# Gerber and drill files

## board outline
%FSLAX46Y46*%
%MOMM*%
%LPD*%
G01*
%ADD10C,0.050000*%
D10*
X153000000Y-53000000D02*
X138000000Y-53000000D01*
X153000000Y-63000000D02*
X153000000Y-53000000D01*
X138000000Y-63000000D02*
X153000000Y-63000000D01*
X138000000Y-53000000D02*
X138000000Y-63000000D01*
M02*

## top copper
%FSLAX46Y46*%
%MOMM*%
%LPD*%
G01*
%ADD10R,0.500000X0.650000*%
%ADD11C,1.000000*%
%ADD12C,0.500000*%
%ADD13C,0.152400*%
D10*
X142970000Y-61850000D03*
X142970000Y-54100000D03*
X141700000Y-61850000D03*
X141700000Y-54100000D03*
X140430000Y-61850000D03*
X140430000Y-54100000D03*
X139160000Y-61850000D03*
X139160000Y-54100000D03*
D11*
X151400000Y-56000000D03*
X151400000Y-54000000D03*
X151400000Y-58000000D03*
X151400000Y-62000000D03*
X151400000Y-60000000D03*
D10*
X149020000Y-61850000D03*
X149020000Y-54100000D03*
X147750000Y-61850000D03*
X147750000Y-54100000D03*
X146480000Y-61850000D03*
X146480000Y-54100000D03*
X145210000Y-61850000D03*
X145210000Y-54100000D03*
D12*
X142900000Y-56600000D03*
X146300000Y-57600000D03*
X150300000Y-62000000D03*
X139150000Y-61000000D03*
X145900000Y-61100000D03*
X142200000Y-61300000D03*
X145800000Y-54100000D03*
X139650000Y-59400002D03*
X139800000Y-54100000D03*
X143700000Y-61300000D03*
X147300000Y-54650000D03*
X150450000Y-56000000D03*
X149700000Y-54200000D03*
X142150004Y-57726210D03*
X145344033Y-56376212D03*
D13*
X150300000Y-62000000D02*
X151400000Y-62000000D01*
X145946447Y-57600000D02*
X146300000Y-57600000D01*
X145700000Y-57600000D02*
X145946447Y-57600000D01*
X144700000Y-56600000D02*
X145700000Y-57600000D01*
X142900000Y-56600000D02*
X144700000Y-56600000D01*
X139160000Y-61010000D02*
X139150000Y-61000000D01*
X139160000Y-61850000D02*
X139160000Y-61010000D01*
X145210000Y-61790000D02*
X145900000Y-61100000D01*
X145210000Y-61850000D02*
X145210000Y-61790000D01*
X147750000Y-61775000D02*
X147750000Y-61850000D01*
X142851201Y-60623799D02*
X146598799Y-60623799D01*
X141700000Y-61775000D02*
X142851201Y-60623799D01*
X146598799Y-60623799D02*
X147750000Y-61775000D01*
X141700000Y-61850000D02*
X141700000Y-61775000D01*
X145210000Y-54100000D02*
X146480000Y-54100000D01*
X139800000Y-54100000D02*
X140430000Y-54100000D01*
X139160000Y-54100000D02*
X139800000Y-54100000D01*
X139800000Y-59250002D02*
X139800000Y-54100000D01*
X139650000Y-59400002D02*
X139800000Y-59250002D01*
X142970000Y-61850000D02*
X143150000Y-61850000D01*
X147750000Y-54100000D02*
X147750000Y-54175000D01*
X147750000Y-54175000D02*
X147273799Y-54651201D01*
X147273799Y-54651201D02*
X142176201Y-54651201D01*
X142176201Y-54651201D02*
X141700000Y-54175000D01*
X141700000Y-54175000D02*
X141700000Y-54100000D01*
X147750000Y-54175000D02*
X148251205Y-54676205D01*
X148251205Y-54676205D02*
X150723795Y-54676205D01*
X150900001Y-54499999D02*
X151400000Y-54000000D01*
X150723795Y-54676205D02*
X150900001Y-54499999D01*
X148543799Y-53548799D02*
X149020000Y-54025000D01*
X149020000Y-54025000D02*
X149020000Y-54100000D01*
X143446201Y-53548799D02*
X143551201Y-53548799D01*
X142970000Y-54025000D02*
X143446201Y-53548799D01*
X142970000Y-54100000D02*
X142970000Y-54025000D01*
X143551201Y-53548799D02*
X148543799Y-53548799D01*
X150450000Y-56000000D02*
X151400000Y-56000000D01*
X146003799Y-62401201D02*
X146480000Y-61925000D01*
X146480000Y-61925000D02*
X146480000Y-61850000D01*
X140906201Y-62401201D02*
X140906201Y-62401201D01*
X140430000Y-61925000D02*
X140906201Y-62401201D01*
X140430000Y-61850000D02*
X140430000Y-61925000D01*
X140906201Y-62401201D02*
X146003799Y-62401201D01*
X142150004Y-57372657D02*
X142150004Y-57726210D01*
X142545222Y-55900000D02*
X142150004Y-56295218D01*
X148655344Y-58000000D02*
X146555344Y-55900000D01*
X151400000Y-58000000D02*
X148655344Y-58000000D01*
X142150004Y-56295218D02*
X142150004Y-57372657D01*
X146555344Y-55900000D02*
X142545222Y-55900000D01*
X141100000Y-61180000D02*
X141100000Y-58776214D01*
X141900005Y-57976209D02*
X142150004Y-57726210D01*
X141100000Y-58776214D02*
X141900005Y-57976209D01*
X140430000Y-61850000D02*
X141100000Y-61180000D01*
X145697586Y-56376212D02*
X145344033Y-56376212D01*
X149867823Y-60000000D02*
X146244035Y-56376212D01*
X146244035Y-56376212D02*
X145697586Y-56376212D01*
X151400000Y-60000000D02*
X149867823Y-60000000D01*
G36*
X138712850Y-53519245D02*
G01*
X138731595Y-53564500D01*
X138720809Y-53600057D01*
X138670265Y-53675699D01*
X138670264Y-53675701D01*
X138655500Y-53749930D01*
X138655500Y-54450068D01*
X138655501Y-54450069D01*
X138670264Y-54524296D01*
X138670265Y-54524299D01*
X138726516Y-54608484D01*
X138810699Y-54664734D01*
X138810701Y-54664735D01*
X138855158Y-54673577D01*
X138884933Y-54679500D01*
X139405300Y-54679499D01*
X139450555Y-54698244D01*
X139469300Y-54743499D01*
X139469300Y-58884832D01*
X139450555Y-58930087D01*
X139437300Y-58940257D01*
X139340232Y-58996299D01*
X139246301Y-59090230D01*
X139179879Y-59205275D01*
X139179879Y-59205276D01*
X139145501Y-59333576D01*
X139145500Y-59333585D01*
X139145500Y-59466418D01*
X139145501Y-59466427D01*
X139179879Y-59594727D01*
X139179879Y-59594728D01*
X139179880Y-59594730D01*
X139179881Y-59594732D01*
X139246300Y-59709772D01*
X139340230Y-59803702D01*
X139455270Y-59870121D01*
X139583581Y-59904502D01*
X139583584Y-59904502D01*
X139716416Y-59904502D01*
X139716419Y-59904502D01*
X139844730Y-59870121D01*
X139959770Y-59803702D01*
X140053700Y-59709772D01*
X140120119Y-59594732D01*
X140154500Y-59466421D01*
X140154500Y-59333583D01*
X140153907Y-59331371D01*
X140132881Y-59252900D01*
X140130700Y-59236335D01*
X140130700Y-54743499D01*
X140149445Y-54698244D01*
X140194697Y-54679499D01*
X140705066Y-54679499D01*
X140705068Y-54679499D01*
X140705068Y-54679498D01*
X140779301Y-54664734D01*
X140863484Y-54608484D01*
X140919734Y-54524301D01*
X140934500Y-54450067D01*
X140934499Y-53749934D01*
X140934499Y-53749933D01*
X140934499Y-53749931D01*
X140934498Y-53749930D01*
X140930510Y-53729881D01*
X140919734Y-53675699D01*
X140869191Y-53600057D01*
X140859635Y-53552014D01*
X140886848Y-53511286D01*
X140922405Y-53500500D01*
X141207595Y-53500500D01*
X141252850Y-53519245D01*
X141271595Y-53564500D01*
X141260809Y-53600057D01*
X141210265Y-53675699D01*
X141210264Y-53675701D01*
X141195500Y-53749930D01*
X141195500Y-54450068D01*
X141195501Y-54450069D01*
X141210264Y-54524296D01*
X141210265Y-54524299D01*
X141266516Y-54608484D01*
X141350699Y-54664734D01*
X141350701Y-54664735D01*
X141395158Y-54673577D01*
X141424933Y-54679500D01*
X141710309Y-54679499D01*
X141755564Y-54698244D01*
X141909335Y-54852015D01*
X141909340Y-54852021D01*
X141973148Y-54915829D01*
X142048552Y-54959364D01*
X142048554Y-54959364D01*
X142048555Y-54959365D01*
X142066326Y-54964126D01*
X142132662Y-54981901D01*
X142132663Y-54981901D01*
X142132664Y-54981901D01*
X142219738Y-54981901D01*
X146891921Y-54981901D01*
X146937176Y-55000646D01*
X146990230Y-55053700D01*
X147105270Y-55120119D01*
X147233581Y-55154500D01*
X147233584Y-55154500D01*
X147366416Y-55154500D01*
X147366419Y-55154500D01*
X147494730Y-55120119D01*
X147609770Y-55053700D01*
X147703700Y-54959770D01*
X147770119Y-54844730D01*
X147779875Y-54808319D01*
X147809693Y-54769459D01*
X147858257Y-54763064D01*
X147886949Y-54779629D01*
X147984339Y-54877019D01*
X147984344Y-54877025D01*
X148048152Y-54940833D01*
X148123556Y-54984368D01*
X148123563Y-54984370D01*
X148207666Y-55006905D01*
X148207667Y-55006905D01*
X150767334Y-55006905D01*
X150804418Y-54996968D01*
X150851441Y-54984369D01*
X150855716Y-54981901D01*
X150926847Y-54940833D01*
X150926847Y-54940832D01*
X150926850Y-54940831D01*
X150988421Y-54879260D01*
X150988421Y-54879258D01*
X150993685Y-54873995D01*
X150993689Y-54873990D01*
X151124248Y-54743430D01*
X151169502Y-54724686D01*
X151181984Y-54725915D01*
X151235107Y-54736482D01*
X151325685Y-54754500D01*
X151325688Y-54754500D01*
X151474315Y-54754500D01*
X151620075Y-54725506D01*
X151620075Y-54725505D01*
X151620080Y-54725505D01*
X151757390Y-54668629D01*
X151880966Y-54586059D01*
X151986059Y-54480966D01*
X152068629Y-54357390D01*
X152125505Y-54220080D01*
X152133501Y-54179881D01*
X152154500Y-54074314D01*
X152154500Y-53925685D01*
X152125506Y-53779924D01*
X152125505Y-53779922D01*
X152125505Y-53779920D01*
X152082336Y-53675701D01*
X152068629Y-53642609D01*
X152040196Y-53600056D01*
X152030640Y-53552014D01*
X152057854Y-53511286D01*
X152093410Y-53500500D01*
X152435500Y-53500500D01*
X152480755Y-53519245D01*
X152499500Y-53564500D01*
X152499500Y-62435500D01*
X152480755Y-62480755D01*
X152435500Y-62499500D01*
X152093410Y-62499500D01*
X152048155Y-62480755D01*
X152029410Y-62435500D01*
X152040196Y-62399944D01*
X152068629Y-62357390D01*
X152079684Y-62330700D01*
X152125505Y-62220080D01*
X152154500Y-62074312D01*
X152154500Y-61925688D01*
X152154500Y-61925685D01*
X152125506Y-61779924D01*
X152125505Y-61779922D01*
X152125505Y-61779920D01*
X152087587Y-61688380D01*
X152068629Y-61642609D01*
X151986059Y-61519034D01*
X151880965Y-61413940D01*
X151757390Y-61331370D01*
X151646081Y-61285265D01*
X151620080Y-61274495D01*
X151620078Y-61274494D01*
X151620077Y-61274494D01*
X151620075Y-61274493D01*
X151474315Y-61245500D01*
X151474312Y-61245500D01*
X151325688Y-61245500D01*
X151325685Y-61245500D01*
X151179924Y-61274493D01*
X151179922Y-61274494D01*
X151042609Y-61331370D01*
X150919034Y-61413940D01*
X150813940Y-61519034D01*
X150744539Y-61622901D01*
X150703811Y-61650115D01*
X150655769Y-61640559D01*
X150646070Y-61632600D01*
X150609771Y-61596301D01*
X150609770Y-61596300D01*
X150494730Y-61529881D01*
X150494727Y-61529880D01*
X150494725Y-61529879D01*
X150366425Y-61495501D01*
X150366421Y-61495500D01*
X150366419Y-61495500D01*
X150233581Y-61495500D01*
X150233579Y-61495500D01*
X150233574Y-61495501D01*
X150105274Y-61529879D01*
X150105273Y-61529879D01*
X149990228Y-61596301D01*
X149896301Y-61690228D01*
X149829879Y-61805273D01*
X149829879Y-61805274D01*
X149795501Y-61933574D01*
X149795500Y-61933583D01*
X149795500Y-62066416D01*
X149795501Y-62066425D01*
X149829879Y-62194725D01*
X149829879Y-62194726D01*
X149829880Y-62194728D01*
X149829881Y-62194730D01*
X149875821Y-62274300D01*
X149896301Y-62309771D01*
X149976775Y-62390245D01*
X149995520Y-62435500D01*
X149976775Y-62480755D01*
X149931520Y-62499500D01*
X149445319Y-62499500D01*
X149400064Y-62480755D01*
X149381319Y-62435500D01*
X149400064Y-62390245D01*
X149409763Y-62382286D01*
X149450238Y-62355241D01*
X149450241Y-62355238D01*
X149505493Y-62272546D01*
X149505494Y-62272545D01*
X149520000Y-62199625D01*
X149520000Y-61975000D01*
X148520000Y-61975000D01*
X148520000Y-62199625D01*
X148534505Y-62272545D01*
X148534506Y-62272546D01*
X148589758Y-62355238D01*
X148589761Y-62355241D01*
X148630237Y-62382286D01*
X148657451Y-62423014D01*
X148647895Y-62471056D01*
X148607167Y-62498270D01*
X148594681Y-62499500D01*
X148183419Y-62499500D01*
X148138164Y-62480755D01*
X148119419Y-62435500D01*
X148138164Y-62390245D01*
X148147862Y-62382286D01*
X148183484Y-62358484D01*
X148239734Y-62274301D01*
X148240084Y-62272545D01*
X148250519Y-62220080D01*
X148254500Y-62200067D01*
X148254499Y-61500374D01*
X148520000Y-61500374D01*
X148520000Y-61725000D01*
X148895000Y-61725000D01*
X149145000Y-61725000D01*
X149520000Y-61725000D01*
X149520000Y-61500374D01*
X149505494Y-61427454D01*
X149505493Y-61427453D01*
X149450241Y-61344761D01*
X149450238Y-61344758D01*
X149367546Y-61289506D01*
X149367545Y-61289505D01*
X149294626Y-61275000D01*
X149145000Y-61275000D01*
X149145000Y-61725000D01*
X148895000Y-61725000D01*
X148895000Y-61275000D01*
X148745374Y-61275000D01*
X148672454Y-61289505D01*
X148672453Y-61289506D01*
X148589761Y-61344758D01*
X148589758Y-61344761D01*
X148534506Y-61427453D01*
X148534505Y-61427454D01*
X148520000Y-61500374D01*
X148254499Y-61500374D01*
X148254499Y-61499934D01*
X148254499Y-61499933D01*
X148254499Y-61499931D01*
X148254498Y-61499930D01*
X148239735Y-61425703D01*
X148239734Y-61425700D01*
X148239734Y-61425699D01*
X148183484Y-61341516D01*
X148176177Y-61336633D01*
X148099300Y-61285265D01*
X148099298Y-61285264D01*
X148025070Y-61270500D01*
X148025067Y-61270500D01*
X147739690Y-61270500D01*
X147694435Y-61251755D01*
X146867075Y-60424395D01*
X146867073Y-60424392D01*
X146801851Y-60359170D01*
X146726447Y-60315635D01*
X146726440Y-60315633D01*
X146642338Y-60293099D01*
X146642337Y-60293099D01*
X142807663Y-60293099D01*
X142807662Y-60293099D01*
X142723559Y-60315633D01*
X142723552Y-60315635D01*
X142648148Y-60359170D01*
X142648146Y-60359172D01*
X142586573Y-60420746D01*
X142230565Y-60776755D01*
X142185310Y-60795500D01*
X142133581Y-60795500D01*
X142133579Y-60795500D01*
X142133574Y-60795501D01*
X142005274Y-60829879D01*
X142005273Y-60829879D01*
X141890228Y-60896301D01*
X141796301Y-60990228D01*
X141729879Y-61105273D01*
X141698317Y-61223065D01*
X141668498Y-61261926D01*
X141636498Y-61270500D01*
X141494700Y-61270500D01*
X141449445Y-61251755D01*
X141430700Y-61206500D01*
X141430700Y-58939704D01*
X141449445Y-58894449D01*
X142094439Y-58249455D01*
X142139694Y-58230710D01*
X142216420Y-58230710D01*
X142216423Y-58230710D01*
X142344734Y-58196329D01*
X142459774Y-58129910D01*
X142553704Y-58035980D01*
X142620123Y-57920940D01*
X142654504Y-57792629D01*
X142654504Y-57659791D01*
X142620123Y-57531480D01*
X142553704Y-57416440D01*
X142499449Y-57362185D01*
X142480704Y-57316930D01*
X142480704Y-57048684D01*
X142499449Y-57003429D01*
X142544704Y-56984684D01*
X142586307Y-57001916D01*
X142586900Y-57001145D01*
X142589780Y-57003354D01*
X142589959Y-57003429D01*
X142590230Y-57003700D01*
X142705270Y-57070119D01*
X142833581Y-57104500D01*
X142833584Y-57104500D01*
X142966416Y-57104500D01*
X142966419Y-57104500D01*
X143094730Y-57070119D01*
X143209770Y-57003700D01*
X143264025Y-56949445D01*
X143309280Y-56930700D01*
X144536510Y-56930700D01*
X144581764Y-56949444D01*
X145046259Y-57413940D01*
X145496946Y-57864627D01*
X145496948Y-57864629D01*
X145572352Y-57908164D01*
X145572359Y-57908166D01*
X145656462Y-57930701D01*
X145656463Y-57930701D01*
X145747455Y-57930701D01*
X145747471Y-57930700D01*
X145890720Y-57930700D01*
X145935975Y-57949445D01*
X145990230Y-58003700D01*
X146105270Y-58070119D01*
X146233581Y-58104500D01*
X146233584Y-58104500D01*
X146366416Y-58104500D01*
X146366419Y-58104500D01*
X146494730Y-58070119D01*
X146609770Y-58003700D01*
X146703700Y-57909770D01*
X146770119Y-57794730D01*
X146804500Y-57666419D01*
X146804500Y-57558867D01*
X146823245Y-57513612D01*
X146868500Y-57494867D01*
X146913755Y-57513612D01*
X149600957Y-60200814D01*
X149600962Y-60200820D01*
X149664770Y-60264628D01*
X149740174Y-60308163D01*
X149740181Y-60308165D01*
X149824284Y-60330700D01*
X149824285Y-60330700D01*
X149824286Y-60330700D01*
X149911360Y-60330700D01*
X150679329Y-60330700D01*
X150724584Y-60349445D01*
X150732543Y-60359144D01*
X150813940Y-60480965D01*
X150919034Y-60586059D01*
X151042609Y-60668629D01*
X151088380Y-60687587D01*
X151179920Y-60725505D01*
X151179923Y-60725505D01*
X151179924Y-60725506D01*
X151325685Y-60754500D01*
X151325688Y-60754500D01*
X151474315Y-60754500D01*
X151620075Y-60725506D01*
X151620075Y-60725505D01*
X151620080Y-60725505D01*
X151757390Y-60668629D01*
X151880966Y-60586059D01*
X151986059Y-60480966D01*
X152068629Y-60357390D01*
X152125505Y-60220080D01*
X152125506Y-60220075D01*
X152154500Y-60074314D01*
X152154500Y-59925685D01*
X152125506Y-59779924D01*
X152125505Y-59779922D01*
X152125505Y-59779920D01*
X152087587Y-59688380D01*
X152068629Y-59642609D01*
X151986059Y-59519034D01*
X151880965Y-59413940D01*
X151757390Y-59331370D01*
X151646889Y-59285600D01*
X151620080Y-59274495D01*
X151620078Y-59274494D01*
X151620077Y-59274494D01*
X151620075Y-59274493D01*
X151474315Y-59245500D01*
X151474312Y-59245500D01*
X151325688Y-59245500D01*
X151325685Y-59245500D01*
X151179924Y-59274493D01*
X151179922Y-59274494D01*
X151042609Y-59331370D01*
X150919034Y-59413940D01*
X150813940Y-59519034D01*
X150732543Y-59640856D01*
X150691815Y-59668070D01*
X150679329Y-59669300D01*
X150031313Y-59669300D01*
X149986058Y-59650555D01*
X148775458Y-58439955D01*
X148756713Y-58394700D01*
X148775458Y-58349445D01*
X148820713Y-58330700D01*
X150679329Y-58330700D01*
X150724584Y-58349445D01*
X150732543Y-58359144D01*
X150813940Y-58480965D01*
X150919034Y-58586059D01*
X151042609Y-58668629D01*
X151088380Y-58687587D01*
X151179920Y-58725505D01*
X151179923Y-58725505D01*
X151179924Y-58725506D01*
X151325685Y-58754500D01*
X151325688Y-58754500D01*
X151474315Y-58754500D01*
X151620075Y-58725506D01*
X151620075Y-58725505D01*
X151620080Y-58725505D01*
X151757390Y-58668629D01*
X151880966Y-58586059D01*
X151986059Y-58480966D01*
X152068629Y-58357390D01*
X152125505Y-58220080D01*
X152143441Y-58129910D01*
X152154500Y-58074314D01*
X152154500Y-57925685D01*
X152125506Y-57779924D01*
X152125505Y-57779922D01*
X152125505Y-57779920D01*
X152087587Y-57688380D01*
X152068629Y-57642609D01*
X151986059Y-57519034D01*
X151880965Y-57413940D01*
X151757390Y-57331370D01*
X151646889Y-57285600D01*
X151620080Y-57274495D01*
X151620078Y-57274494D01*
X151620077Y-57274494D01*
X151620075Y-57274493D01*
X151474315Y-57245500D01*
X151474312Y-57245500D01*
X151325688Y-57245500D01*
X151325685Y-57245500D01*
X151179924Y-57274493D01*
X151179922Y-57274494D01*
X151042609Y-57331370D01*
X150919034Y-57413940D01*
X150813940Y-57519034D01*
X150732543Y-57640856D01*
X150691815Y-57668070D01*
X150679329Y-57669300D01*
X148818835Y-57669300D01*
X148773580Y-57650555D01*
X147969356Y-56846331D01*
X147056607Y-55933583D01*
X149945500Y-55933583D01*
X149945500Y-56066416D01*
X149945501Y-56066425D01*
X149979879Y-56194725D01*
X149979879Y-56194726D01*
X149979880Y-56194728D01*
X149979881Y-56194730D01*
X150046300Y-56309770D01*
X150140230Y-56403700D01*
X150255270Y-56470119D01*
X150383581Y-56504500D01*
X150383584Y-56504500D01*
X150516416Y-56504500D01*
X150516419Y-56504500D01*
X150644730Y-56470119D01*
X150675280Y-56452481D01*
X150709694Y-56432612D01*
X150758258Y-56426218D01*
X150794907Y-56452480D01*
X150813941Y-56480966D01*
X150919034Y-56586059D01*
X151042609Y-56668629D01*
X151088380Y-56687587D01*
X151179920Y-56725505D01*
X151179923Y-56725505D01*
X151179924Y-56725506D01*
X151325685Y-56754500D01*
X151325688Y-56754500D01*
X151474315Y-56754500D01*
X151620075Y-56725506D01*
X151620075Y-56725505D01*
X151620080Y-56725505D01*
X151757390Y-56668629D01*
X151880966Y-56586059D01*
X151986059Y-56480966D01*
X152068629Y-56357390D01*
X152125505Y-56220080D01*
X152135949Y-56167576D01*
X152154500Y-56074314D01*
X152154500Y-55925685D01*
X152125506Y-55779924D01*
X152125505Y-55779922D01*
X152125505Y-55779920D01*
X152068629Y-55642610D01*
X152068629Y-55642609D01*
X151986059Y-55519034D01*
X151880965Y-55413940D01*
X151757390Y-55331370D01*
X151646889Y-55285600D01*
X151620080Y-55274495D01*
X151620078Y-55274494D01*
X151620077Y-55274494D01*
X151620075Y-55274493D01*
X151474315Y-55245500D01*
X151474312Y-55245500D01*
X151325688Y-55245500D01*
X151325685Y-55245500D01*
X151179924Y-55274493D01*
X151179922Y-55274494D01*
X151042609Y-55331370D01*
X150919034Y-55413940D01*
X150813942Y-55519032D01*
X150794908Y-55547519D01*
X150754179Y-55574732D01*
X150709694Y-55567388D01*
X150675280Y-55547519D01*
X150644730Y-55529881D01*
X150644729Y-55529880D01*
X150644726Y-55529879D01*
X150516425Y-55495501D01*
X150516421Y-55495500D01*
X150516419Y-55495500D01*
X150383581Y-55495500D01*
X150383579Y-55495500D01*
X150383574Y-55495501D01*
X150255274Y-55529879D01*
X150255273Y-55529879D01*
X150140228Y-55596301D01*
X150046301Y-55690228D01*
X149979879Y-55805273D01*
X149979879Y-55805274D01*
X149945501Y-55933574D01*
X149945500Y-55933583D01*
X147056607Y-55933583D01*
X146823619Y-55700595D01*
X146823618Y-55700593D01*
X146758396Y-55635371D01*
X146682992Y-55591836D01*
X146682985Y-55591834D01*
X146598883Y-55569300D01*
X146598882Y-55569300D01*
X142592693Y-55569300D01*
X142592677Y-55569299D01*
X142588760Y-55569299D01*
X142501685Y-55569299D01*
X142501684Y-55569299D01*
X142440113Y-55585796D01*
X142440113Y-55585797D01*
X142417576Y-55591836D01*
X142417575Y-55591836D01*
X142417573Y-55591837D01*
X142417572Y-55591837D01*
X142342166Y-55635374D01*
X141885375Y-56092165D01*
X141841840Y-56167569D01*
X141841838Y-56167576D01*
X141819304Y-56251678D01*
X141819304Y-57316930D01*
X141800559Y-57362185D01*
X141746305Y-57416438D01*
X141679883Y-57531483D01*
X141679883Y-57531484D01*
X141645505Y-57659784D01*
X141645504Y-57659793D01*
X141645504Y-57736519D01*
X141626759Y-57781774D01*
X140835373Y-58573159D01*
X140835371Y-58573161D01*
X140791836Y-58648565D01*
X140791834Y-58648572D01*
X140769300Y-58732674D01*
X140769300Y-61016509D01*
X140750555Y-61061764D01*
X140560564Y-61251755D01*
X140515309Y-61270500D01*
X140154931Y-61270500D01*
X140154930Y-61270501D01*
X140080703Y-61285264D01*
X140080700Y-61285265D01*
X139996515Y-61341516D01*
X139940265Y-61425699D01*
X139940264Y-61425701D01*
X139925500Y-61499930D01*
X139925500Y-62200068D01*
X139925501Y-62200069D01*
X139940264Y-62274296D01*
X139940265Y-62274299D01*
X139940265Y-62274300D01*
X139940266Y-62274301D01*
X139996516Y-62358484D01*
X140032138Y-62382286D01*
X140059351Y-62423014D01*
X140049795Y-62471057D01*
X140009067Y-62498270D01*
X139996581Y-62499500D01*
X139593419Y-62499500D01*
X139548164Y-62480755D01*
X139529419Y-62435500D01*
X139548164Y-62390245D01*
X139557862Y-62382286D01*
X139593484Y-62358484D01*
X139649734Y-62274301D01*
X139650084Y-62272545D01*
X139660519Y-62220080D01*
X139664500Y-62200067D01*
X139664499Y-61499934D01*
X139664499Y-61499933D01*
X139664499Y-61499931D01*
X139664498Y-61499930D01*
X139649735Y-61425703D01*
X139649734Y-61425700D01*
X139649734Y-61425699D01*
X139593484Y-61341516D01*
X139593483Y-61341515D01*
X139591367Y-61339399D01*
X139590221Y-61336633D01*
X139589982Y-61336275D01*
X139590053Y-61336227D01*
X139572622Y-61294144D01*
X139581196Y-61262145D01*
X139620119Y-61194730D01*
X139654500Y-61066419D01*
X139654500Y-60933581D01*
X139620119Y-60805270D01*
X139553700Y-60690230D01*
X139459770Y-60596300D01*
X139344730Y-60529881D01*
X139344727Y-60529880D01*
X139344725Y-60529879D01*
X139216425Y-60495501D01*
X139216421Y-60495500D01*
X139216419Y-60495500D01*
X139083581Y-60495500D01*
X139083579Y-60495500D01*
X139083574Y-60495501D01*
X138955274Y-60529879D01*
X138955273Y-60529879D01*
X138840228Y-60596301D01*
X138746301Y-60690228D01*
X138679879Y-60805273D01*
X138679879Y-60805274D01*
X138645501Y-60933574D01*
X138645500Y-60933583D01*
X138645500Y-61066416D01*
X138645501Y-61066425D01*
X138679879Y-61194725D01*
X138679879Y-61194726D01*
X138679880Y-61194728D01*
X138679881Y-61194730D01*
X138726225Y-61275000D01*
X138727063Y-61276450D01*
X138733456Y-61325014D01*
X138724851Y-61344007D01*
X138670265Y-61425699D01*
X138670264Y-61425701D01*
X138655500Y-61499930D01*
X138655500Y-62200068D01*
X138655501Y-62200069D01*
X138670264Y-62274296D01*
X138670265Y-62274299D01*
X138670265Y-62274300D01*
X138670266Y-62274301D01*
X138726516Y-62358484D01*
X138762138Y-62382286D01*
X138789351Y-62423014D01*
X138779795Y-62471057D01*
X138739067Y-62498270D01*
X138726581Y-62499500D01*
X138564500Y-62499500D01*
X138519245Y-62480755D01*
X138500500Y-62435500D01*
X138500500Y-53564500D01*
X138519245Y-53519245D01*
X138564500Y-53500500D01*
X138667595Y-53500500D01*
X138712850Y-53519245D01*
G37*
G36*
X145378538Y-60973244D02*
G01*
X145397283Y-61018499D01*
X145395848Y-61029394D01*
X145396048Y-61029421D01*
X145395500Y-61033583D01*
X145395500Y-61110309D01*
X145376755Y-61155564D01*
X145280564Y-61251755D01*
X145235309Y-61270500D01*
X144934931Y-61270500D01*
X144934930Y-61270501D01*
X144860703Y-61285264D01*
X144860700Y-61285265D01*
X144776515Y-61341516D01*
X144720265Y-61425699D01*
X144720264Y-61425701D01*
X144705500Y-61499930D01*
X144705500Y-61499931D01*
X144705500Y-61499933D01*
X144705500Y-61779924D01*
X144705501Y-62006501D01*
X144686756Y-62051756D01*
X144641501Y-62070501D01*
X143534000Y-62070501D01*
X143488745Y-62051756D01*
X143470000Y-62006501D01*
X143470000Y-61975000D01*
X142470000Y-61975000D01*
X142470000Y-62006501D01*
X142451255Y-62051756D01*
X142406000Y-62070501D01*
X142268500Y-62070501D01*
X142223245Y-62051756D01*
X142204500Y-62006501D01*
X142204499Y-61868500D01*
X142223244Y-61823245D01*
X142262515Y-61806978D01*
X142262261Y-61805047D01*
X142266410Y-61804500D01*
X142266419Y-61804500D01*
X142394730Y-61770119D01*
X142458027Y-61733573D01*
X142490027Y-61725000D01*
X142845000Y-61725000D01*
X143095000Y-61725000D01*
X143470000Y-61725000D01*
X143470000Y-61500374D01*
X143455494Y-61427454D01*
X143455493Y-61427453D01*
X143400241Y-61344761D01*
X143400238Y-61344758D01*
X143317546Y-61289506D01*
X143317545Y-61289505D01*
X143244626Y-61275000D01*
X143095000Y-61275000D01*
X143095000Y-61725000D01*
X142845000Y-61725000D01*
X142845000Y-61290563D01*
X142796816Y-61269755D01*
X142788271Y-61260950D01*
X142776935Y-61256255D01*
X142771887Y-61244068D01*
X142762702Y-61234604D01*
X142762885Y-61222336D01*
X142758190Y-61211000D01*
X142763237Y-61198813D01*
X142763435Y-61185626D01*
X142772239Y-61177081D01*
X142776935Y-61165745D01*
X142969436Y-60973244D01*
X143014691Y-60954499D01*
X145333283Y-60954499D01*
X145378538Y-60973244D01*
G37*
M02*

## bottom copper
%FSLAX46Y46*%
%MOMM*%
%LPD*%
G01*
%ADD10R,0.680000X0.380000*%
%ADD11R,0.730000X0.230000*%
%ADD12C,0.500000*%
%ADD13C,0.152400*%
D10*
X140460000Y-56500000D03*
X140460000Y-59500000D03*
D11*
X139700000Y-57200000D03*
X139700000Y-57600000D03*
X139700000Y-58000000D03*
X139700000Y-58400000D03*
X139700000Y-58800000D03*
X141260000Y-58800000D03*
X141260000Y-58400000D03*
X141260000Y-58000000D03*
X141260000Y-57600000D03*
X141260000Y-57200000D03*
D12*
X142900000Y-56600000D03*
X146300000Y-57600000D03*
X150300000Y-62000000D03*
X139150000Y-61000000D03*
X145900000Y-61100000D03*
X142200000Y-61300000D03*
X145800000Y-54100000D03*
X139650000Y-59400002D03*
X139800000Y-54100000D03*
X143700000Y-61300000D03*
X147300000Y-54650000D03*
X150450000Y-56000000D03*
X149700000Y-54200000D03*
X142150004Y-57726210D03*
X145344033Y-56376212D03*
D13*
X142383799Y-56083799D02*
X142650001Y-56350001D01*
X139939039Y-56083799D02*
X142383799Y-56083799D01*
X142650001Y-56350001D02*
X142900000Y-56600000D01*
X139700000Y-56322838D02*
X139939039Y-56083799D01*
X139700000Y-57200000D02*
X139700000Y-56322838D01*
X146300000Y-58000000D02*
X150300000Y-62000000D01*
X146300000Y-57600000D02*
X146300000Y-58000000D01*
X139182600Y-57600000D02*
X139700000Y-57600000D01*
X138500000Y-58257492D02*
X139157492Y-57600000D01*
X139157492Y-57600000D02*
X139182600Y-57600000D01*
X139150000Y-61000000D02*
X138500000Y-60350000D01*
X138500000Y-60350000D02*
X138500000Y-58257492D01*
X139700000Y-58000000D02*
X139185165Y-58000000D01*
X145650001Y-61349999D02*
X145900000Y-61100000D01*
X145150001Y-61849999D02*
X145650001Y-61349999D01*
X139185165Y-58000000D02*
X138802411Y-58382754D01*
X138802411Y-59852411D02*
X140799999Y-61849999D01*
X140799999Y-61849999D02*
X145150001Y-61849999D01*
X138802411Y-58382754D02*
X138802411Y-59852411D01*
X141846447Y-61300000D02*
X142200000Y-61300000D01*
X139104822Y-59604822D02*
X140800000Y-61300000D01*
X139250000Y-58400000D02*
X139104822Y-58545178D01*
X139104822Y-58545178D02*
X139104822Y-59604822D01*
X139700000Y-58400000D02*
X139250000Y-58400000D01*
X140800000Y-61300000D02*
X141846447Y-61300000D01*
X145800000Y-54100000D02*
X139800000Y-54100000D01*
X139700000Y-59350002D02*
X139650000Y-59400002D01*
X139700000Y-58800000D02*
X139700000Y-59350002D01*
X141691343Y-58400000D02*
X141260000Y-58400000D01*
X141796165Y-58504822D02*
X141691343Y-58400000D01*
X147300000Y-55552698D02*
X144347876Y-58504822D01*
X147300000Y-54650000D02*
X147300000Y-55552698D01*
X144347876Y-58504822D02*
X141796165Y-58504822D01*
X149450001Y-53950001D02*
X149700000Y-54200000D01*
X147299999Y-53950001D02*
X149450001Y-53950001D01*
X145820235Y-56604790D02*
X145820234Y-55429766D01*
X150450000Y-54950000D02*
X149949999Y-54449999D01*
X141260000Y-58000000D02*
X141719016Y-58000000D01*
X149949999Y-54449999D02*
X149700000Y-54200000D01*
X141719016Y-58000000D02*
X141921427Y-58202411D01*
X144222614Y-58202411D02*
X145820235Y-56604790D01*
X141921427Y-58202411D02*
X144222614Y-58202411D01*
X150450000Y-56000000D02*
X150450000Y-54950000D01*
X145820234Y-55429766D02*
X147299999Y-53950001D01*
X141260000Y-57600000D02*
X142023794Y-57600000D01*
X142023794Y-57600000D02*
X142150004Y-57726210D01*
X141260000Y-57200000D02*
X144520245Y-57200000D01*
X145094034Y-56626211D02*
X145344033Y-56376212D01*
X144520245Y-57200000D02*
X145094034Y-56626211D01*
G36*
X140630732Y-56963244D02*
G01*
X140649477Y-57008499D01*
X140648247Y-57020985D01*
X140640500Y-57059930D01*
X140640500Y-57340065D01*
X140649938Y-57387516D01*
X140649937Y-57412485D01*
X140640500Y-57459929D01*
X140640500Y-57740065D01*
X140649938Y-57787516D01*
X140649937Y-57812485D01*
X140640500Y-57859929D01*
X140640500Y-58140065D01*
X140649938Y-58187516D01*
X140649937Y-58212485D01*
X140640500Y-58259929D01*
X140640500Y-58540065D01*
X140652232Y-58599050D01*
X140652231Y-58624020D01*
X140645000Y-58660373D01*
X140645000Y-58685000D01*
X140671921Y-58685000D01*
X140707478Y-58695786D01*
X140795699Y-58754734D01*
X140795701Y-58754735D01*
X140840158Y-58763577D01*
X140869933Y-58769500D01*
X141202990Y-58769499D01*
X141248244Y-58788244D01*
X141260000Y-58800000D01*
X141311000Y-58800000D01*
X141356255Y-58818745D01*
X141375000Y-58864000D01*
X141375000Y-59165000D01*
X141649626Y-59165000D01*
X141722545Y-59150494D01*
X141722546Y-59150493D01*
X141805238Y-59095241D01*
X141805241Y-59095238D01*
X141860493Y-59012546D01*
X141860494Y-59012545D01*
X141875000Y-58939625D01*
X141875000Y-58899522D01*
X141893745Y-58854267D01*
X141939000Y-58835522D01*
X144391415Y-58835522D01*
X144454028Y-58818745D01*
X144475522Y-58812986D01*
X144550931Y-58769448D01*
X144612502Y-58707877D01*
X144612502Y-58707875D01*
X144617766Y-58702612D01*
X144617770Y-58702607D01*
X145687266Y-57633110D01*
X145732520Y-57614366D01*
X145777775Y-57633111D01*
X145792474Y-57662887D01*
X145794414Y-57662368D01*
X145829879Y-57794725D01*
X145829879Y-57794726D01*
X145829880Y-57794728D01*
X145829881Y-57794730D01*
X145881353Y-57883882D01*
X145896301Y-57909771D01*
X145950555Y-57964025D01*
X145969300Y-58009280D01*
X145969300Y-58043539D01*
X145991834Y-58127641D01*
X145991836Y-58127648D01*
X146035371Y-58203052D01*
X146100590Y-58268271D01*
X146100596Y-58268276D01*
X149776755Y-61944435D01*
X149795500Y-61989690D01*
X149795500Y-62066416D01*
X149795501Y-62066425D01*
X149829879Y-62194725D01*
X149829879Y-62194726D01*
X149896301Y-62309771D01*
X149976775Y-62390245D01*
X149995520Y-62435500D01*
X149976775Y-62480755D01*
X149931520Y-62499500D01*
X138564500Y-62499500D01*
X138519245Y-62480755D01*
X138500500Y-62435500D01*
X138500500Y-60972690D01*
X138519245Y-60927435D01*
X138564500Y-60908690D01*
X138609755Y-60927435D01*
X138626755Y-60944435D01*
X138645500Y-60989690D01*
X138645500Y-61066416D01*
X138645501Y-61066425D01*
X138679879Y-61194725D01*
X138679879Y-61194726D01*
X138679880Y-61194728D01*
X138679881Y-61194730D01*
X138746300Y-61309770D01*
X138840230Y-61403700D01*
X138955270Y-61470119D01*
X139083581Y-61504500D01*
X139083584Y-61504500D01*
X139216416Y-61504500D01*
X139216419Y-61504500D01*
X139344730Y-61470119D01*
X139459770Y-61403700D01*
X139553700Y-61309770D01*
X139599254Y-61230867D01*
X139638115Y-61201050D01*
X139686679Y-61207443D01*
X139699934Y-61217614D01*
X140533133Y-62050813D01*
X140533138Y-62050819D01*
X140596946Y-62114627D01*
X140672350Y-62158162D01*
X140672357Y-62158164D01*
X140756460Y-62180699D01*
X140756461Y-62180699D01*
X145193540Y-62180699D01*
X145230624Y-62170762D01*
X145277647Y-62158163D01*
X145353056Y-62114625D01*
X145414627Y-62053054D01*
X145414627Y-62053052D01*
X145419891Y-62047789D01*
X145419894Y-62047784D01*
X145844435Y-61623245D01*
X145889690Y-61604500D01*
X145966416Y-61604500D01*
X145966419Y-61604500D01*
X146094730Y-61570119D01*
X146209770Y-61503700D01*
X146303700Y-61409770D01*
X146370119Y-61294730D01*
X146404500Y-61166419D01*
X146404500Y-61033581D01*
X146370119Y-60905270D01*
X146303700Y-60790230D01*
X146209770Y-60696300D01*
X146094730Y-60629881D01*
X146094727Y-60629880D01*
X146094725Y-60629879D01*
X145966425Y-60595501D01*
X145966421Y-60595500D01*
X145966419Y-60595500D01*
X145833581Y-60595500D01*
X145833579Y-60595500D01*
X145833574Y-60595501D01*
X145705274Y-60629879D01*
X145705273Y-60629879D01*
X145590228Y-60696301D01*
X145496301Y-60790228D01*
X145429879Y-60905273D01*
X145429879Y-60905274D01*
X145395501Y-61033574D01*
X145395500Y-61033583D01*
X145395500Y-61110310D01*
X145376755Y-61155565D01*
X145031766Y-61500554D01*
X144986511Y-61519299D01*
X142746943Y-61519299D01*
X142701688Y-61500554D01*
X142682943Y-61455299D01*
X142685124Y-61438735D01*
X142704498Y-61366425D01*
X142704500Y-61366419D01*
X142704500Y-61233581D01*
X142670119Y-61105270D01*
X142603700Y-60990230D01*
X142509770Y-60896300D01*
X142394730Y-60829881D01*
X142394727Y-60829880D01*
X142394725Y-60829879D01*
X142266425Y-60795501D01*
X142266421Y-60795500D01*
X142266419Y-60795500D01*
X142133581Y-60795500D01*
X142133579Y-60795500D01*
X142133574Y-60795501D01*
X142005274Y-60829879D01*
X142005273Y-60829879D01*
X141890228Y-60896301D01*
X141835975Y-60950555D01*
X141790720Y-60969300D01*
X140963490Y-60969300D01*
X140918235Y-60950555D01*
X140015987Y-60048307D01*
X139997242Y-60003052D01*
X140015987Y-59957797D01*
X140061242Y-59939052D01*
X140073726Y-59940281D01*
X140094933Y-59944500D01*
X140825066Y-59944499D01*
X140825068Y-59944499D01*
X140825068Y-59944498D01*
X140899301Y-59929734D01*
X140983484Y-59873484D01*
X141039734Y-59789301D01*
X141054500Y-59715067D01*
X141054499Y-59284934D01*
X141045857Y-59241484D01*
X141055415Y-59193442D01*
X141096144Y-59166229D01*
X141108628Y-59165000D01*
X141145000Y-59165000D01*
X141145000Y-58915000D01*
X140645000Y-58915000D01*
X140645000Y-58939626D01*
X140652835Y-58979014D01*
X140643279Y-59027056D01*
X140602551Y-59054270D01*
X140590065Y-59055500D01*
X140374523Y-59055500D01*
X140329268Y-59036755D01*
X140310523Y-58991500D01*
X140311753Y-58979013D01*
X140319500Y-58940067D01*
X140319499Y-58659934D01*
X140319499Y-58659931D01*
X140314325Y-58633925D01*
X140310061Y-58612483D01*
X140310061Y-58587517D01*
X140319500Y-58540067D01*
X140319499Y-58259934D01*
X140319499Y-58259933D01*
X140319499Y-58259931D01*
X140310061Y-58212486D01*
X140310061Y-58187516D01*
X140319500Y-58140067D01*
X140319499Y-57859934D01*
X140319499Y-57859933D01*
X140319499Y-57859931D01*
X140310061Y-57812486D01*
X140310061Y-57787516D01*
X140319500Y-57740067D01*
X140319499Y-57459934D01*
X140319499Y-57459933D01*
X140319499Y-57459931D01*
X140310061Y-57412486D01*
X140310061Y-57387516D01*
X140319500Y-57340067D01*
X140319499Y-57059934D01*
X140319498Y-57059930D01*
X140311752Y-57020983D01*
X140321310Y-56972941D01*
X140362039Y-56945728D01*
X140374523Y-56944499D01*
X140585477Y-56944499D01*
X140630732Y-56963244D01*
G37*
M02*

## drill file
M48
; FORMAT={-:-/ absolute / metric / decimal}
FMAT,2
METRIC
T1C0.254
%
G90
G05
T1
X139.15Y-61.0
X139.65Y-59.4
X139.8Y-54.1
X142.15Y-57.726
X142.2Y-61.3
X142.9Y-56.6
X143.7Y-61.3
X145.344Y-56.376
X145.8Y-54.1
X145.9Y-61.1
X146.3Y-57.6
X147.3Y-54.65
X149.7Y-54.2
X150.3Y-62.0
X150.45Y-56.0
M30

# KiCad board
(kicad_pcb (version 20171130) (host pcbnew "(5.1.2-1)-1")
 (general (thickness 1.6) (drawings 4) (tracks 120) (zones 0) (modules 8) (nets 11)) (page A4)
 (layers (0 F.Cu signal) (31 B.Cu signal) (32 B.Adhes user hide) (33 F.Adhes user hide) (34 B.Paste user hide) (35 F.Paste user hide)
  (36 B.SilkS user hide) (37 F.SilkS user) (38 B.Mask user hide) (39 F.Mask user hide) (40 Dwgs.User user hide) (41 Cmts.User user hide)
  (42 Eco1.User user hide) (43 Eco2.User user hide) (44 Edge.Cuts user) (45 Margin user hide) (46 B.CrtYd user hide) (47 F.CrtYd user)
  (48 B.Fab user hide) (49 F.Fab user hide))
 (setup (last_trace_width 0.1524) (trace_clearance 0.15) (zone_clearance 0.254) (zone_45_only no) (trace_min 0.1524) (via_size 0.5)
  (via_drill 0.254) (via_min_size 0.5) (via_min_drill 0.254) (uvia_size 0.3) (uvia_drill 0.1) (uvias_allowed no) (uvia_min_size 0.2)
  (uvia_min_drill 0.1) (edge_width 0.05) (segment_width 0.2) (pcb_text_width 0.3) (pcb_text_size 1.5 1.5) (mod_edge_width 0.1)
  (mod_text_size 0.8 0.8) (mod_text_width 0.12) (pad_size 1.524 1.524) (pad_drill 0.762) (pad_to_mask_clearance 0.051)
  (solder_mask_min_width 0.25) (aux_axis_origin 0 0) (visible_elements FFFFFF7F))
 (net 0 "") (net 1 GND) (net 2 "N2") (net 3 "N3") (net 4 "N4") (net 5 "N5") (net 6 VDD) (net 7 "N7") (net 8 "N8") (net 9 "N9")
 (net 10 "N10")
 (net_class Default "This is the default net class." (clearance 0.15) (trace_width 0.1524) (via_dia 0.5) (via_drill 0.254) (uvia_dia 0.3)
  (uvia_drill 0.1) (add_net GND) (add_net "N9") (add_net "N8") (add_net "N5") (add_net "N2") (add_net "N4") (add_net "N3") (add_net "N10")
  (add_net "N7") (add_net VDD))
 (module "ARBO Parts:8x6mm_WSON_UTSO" (layer F.Cu) (at 141.065 57.975)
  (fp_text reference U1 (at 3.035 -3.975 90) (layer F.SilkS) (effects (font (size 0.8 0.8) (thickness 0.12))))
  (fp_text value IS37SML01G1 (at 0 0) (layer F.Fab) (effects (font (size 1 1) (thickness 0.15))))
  (pad 4 smd rect (at 1.905 3.875) (size 0.5 0.65) (layers F.Cu F.Paste F.Mask) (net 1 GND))
  (pad 5 smd rect (at 1.905 -3.875) (size 0.5 0.65) (layers F.Cu F.Paste F.Mask) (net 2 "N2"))
  (pad 3 smd rect (at 0.635 3.875) (size 0.5 0.65) (layers F.Cu F.Paste F.Mask) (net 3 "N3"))
  (pad 6 smd rect (at 0.635 -3.875) (size 0.5 0.65) (layers F.Cu F.Paste F.Mask) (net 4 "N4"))
  (pad 2 smd rect (at -0.635 3.875) (size 0.5 0.65) (layers F.Cu F.Paste F.Mask) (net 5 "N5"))
  (pad 7 smd rect (at -0.635 -3.875) (size 0.5 0.65) (layers F.Cu F.Paste F.Mask) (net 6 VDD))
  (pad 1 smd rect (at -1.905 3.875) (size 0.5 0.65) (layers F.Cu F.Paste F.Mask) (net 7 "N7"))
  (pad 8 smd rect (at -1.905 -3.875) (size 0.5 0.65) (layers F.Cu F.Paste F.Mask) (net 6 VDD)))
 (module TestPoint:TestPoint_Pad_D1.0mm (layer F.Cu) (at 151.4 56)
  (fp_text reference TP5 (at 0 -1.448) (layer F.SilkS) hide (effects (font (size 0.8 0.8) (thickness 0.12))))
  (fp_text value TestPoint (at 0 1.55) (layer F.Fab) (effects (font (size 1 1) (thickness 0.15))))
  (pad 1 smd circle (at 0 0) (size 1 1) (layers F.Cu F.Mask) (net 2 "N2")))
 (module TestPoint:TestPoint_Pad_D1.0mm (layer F.Cu) (at 151.4 54)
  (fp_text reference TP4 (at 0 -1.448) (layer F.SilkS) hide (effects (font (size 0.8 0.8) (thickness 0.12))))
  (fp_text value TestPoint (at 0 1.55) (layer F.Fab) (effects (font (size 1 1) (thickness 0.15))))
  (pad 1 smd circle (at 0 0) (size 1 1) (layers F.Cu F.Mask) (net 4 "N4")))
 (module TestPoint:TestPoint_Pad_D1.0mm (layer F.Cu) (at 151.4 58)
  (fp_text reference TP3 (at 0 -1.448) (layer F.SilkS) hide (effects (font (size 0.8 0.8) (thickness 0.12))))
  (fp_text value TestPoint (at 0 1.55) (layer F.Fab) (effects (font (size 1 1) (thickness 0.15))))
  (pad 1 smd circle (at 0 0) (size 1 1) (layers F.Cu F.Mask) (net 5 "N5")))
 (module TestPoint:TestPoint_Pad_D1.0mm (layer F.Cu) (at 151.4 62)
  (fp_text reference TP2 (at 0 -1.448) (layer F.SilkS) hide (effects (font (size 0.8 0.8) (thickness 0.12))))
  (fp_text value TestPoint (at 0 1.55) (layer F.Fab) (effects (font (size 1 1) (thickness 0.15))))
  (pad 1 smd circle (at 0 0) (size 1 1) (layers F.Cu F.Mask) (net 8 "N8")))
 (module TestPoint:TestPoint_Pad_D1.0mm (layer F.Cu) (at 151.4 60)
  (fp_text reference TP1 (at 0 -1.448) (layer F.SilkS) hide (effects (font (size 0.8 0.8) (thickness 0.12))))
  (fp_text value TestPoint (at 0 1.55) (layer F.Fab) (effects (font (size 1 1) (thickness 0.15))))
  (pad 1 smd circle (at 0 0) (size 1 1) (layers F.Cu F.Mask) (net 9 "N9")))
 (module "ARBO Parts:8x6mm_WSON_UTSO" (layer F.Cu) (at 147.115 57.975)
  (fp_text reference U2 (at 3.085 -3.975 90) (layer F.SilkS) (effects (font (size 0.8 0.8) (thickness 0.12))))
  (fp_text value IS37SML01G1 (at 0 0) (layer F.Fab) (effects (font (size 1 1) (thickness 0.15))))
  (pad 4 smd rect (at 1.905 3.875) (size 0.5 0.65) (layers F.Cu F.Paste F.Mask) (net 1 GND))
  (pad 5 smd rect (at 1.905 -3.875) (size 0.5 0.65) (layers F.Cu F.Paste F.Mask) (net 2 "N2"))
  (pad 3 smd rect (at 0.635 3.875) (size 0.5 0.65) (layers F.Cu F.Paste F.Mask) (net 3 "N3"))
  (pad 6 smd rect (at 0.635 -3.875) (size 0.5 0.65) (layers F.Cu F.Paste F.Mask) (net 4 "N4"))
  (pad 2 smd rect (at -0.635 3.875) (size 0.5 0.65) (layers F.Cu F.Paste F.Mask) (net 5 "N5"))
  (pad 7 smd rect (at -0.635 -3.875) (size 0.5 0.65) (layers F.Cu F.Paste F.Mask) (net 6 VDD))
  (pad 1 smd rect (at -1.905 3.875) (size 0.5 0.65) (layers F.Cu F.Paste F.Mask) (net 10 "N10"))
  (pad 8 smd rect (at -1.905 -3.875) (size 0.5 0.65) (layers F.Cu F.Paste F.Mask) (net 6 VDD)))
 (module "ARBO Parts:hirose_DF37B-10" (layer B.Cu) (at 141.26 58 270)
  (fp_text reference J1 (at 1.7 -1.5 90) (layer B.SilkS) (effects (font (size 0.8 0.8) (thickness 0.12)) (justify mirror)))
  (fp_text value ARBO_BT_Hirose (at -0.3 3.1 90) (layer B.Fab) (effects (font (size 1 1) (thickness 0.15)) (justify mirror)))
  (pad 12 smd rect (at -1.5 0.8 270) (size 0.38 0.68) (layers B.Cu B.Paste B.Mask))
  (pad 11 smd rect (at 1.5 0.8 270) (size 0.38 0.68) (layers B.Cu B.Paste B.Mask))
  (pad 10 smd rect (at -0.8 1.56 270) (size 0.23 0.73) (layers B.Cu B.Paste B.Mask) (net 8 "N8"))
  (pad 9 smd rect (at -0.4 1.56 270) (size 0.23 0.73) (layers B.Cu B.Paste B.Mask) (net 7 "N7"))
  (pad 8 smd rect (at 0 1.56 270) (size 0.23 0.73) (layers B.Cu B.Paste B.Mask) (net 10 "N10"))
  (pad 7 smd rect (at 0.4 1.56 270) (size 0.23 0.73) (layers B.Cu B.Paste B.Mask) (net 3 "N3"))
  (pad 6 smd rect (at 0.8 1.56 270) (size 0.23 0.73) (layers B.Cu B.Paste B.Mask) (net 6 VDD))
  (pad 5 smd rect (at 0.8 0 270) (size 0.23 0.73) (layers B.Cu B.Paste B.Mask) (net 1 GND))
  (pad 4 smd rect (at 0.4 0 270) (size 0.23 0.73) (layers B.Cu B.Paste B.Mask) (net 4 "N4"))
  (pad 3 smd rect (at 0 0 270) (size 0.23 0.73) (layers B.Cu B.Paste B.Mask) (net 2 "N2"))
  (pad 2 smd rect (at -0.4 0 270) (size 0.23 0.73) (layers B.Cu B.Paste B.Mask) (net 5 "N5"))
  (pad 1 smd rect (at -0.8 0 270) (size 0.23 0.73) (layers B.Cu B.Paste B.Mask) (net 9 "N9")))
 (gr_line (start 153 53) (end 138 53) (layer Edge.Cuts) (width 0.05))
 (gr_line (start 153 63) (end 153 53) (layer Edge.Cuts) (width 0.05))
 (gr_line (start 138 63) (end 153 63) (layer Edge.Cuts) (width 0.05))
 (gr_line (start 138 53) (end 138 63) (layer Edge.Cuts) (width 0.05))
 (via (at 142.9 56.6) (size 0.5) (drill 0.254) (layers F.Cu B.Cu) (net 8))
 (via (at 146.3 57.6) (size 0.5) (drill 0.254) (layers F.Cu B.Cu) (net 8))
 (via (at 150.3 62) (size 0.5) (drill 0.254) (layers F.Cu B.Cu) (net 8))
 (segment (start 150.3 62) (end 151.4 62) (width 0.1524) (layer F.Cu) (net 8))
 (segment (start 145.946447 57.6) (end 146.3 57.6) (width 0.1524) (layer F.Cu) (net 8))
 (segment (start 145.7 57.6) (end 145.946447 57.6) (width 0.1524) (layer F.Cu) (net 8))
 (segment (start 144.7 56.6) (end 145.7 57.6) (width 0.1524) (layer F.Cu) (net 8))
 (segment (start 142.9 56.6) (end 144.7 56.6) (width 0.1524) (layer F.Cu) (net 8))
 (segment (start 142.383799 56.083799) (end 142.650001 56.350001) (width 0.1524) (layer B.Cu) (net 8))
 (segment (start 139.939039 56.083799) (end 142.383799 56.083799) (width 0.1524) (layer B.Cu) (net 8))
 (segment (start 142.650001 56.350001) (end 142.9 56.6) (width 0.1524) (layer B.Cu) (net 8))
 (segment (start 139.7 56.322838) (end 139.939039 56.083799) (width 0.1524) (layer B.Cu) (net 8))
 (segment (start 139.7 57.2) (end 139.7 56.322838) (width 0.1524) (layer B.Cu) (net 8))
 (segment (start 146.3 58) (end 150.3 62) (width 0.1524) (layer B.Cu) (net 8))
 (segment (start 146.3 57.6) (end 146.3 58) (width 0.1524) (layer B.Cu) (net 8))
 (via (at 139.15 61) (size 0.5) (drill 0.254) (layers F.Cu B.Cu) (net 7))
 (segment (start 139.16 61.01) (end 139.15 61) (width 0.1524) (layer F.Cu) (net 7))
 (segment (start 139.16 61.85) (end 139.16 61.01) (width 0.1524) (layer F.Cu) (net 7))
 (segment (start 139.1826 57.6) (end 139.7 57.6) (width 0.1524) (layer B.Cu) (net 7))
 (segment (start 138.5 58.257492) (end 139.157492 57.6) (width 0.1524) (layer B.Cu) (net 7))
 (segment (start 139.157492 57.6) (end 139.1826 57.6) (width 0.1524) (layer B.Cu) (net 7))
 (segment (start 139.15 61) (end 138.5 60.35) (width 0.1524) (layer B.Cu) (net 7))
 (segment (start 138.5 60.35) (end 138.5 58.257492) (width 0.1524) (layer B.Cu) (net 7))
 (via (at 145.9 61.1) (size 0.5) (drill 0.254) (layers F.Cu B.Cu) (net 10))
 (segment (start 139.7 58) (end 139.185165 58) (width 0.1524) (layer B.Cu) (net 10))
 (segment (start 145.650001 61.349999) (end 145.9 61.1) (width 0.1524) (layer B.Cu) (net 10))
 (segment (start 145.150001 61.849999) (end 145.650001 61.349999) (width 0.1524) (layer B.Cu) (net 10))
 (segment (start 139.185165 58) (end 138.802411 58.382754) (width 0.1524) (layer B.Cu) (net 10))
 (segment (start 138.802411 59.852411) (end 140.799999 61.849999) (width 0.1524) (layer B.Cu) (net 10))
 (segment (start 140.799999 61.849999) (end 145.150001 61.849999) (width 0.1524) (layer B.Cu) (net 10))
 (segment (start 138.802411 58.382754) (end 138.802411 59.852411) (width 0.1524) (layer B.Cu) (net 10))
 (segment (start 145.21 61.79) (end 145.9 61.1) (width 0.1524) (layer F.Cu) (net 10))
 (segment (start 145.21 61.85) (end 145.21 61.79) (width 0.1524) (layer F.Cu) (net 10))
 (via (at 142.2 61.3) (size 0.5) (drill 0.254) (layers F.Cu B.Cu) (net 3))
 (segment (start 141.846447 61.3) (end 142.2 61.3) (width 0.1524) (layer B.Cu) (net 3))
 (segment (start 139.104822 59.604822) (end 140.8 61.3) (width 0.1524) (layer B.Cu) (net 3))
 (segment (start 139.25 58.4) (end 139.104822 58.545178) (width 0.1524) (layer B.Cu) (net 3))
 (segment (start 139.104822 58.545178) (end 139.104822 59.604822) (width 0.1524) (layer B.Cu) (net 3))
 (segment (start 139.7 58.4) (end 139.25 58.4) (width 0.1524) (layer B.Cu) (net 3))
 (segment (start 140.8 61.3) (end 141.846447 61.3) (width 0.1524) (layer B.Cu) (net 3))
 (segment (start 147.75 61.775) (end 147.75 61.85) (width 0.1524) (layer F.Cu) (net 3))
 (segment (start 142.851201 60.623799) (end 146.598799 60.623799) (width 0.1524) (layer F.Cu) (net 3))
 (segment (start 141.7 61.775) (end 142.851201 60.623799) (width 0.1524) (layer F.Cu) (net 3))
 (segment (start 146.598799 60.623799) (end 147.75 61.775) (width 0.1524) (layer F.Cu) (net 3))
 (segment (start 141.7 61.85) (end 141.7 61.775) (width 0.1524) (layer F.Cu) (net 3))
 (via (at 145.8 54.1) (size 0.5) (drill 0.254) (layers F.Cu B.Cu) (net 6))
 (segment (start 145.21 54.1) (end 146.48 54.1) (width 0.1524) (layer F.Cu) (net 6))
 (segment (start 145.8 54.1) (end 139.8 54.1) (width 0.1524) (layer B.Cu) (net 6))
 (segment (start 139.7 59.350002) (end 139.65 59.400002) (width 0.1524) (layer B.Cu) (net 6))
 (via (at 139.65 59.400002) (size 0.5) (drill 0.254) (layers F.Cu B.Cu) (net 6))
 (segment (start 139.7 58.8) (end 139.7 59.350002) (width 0.1524) (layer B.Cu) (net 6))
 (segment (start 139.8 54.1) (end 140.43 54.1) (width 0.1524) (layer F.Cu) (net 6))
 (segment (start 139.16 54.1) (end 139.8 54.1) (width 0.1524) (layer F.Cu) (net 6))
 (via (at 139.8 54.1) (size 0.5) (drill 0.254) (layers F.Cu B.Cu) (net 6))
 (segment (start 139.8 59.250002) (end 139.8 54.1) (width 0.1524) (layer F.Cu) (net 6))
 (segment (start 139.65 59.400002) (end 139.8 59.250002) (width 0.1524) (layer F.Cu) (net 6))
 (via (at 143.7 61.3) (size 0.5) (drill 0.254) (layers F.Cu B.Cu) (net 1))
 (segment (start 142.97 61.85) (end 143.15 61.85) (width 0.1524) (layer F.Cu) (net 1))
 (via (at 147.3 54.65) (size 0.5) (drill 0.254) (layers F.Cu B.Cu) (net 4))
 (segment (start 147.75 54.1) (end 147.75 54.175) (width 0.1524) (layer F.Cu) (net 4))
 (segment (start 147.75 54.175) (end 147.273799 54.651201) (width 0.1524) (layer F.Cu) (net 4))
 (segment (start 147.273799 54.651201) (end 142.176201 54.651201) (width 0.1524) (layer F.Cu) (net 4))
 (segment (start 142.176201 54.651201) (end 141.7 54.175) (width 0.1524) (layer F.Cu) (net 4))
 (segment (start 141.7 54.175) (end 141.7 54.1) (width 0.1524) (layer F.Cu) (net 4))
 (segment (start 141.691343 58.4) (end 141.26 58.4) (width 0.1524) (layer B.Cu) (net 4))
 (segment (start 141.796165 58.504822) (end 141.691343 58.4) (width 0.1524) (layer B.Cu) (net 4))
 (segment (start 147.3 55.552698) (end 144.347876 58.504822) (width 0.1524) (layer B.Cu) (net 4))
 (segment (start 147.3 54.65) (end 147.3 55.552698) (width 0.1524) (layer B.Cu) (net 4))
 (segment (start 144.347876 58.504822) (end 141.796165 58.504822) (width 0.1524) (layer B.Cu) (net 4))
 (segment (start 147.75 54.175) (end 148.251205 54.676205) (width 0.1524) (layer F.Cu) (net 4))
 (segment (start 148.251205 54.676205) (end 150.723795 54.676205) (width 0.1524) (layer F.Cu) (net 4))
 (segment (start 150.900001 54.499999) (end 151.4 54) (width 0.1524) (layer F.Cu) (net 4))
 (segment (start 150.723795 54.676205) (end 150.900001 54.499999) (width 0.1524) (layer F.Cu) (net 4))
 (segment (start 148.543799 53.548799) (end 149.02 54.025) (width 0.1524) (layer F.Cu) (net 2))
 (segment (start 149.02 54.025) (end 149.02 54.1) (width 0.1524) (layer F.Cu) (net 2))
 (segment (start 143.446201 53.548799) (end 143.551201 53.548799) (width 0.1524) (layer F.Cu) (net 2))
 (segment (start 142.97 54.025) (end 143.446201 53.548799) (width 0.1524) (layer F.Cu) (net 2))
 (segment (start 142.97 54.1) (end 142.97 54.025) (width 0.1524) (layer F.Cu) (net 2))
 (segment (start 143.551201 53.548799) (end 148.543799 53.548799) (width 0.1524) (layer F.Cu) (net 2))
 (via (at 150.45 56) (size 0.5) (drill 0.254) (layers F.Cu B.Cu) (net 2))
 (segment (start 150.45 56) (end 151.4 56) (width 0.1524) (layer F.Cu) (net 2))
 (segment (start 149.450001 53.950001) (end 149.7 54.2) (width 0.1524) (layer B.Cu) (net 2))
 (segment (start 147.299999 53.950001) (end 149.450001 53.950001) (width 0.1524) (layer B.Cu) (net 2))
 (via (at 149.7 54.2) (size 0.5) (drill 0.254) (layers F.Cu B.Cu) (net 2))
 (segment (start 145.820235 56.60479) (end 145.820234 55.429766) (width 0.1524) (layer B.Cu) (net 2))
 (segment (start 150.45 54.95) (end 149.949999 54.449999) (width 0.1524) (layer B.Cu) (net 2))
 (segment (start 141.26 58) (end 141.719016 58) (width 0.1524) (layer B.Cu) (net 2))
 (segment (start 149.949999 54.449999) (end 149.7 54.2) (width 0.1524) (layer B.Cu) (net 2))
 (segment (start 141.719016 58) (end 141.921427 58.202411) (width 0.1524) (layer B.Cu) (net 2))
 (segment (start 144.222614 58.202411) (end 145.820235 56.60479) (width 0.1524) (layer B.Cu) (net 2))
 (segment (start 141.921427 58.202411) (end 144.222614 58.202411) (width 0.1524) (layer B.Cu) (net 2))
 (segment (start 150.45 56) (end 150.45 54.95) (width 0.1524) (layer B.Cu) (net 2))
 (segment (start 145.820234 55.429766) (end 147.299999 53.950001) (width 0.1524) (layer B.Cu) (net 2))
 (segment (start 146.003799 62.401201) (end 146.48 61.925) (width 0.1524) (layer F.Cu) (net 5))
 (segment (start 146.48 61.925) (end 146.48 61.85) (width 0.1524) (layer F.Cu) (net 5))
 (segment (start 140.906201 62.401201) (end 140.906201 62.401201) (width 0.1524) (layer F.Cu) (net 5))
 (segment (start 140.43 61.925) (end 140.906201 62.401201) (width 0.1524) (layer F.Cu) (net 5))
 (segment (start 140.43 61.85) (end 140.43 61.925) (width 0.1524) (layer F.Cu) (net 5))
 (segment (start 140.906201 62.401201) (end 146.003799 62.401201) (width 0.1524) (layer F.Cu) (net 5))
 (segment (start 141.26 57.6) (end 142.023794 57.6) (width 0.1524) (layer B.Cu) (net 5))
 (segment (start 142.023794 57.6) (end 142.150004 57.72621) (width 0.1524) (layer B.Cu) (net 5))
 (via (at 142.150004 57.72621) (size 0.5) (drill 0.254) (layers F.Cu B.Cu) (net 5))
 (segment (start 142.150004 57.372657) (end 142.150004 57.72621) (width 0.1524) (layer F.Cu) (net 5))
 (segment (start 142.545222 55.9) (end 142.150004 56.295218) (width 0.1524) (layer F.Cu) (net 5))
 (segment (start 148.655344 58) (end 146.555344 55.9) (width 0.1524) (layer F.Cu) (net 5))
 (segment (start 151.4 58) (end 148.655344 58) (width 0.1524) (layer F.Cu) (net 5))
 (segment (start 142.150004 56.295218) (end 142.150004 57.372657) (width 0.1524) (layer F.Cu) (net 5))
 (segment (start 146.555344 55.9) (end 142.545222 55.9) (width 0.1524) (layer F.Cu) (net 5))
 (segment (start 141.1 61.18) (end 141.1 58.776214) (width 0.1524) (layer F.Cu) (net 5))
 (segment (start 141.900005 57.976209) (end 142.150004 57.72621) (width 0.1524) (layer F.Cu) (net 5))
 (segment (start 141.1 58.776214) (end 141.900005 57.976209) (width 0.1524) (layer F.Cu) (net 5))
 (segment (start 140.43 61.85) (end 141.1 61.18) (width 0.1524) (layer F.Cu) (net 5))
 (segment (start 145.697586 56.376212) (end 145.344033 56.376212) (width 0.1524) (layer F.Cu) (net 9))
 (via (at 145.344033 56.376212) (size 0.5) (drill 0.254) (layers F.Cu B.Cu) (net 9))
 (segment (start 149.867823 60) (end 146.244035 56.376212) (width 0.1524) (layer F.Cu) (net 9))
 (segment (start 146.244035 56.376212) (end 145.697586 56.376212) (width 0.1524) (layer F.Cu) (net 9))
 (segment (start 141.26 57.2) (end 144.520245 57.2) (width 0.1524) (layer B.Cu) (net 9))
 (segment (start 151.4 60) (end 149.867823 60) (width 0.1524) (layer F.Cu) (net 9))
 (segment (start 145.094034 56.626211) (end 145.344033 56.376212) (width 0.1524) (layer B.Cu) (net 9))
 (segment (start 144.520245 57.2) (end 145.094034 56.626211) (width 0.1524) (layer B.Cu) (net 9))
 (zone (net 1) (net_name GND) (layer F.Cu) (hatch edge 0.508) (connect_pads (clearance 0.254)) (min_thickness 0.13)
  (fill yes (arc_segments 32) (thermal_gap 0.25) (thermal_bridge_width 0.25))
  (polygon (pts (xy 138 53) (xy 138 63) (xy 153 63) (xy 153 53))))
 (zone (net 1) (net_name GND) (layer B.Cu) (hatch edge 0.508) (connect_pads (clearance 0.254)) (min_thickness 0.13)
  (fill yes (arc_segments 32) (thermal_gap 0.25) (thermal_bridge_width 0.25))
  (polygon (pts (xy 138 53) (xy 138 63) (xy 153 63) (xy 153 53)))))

